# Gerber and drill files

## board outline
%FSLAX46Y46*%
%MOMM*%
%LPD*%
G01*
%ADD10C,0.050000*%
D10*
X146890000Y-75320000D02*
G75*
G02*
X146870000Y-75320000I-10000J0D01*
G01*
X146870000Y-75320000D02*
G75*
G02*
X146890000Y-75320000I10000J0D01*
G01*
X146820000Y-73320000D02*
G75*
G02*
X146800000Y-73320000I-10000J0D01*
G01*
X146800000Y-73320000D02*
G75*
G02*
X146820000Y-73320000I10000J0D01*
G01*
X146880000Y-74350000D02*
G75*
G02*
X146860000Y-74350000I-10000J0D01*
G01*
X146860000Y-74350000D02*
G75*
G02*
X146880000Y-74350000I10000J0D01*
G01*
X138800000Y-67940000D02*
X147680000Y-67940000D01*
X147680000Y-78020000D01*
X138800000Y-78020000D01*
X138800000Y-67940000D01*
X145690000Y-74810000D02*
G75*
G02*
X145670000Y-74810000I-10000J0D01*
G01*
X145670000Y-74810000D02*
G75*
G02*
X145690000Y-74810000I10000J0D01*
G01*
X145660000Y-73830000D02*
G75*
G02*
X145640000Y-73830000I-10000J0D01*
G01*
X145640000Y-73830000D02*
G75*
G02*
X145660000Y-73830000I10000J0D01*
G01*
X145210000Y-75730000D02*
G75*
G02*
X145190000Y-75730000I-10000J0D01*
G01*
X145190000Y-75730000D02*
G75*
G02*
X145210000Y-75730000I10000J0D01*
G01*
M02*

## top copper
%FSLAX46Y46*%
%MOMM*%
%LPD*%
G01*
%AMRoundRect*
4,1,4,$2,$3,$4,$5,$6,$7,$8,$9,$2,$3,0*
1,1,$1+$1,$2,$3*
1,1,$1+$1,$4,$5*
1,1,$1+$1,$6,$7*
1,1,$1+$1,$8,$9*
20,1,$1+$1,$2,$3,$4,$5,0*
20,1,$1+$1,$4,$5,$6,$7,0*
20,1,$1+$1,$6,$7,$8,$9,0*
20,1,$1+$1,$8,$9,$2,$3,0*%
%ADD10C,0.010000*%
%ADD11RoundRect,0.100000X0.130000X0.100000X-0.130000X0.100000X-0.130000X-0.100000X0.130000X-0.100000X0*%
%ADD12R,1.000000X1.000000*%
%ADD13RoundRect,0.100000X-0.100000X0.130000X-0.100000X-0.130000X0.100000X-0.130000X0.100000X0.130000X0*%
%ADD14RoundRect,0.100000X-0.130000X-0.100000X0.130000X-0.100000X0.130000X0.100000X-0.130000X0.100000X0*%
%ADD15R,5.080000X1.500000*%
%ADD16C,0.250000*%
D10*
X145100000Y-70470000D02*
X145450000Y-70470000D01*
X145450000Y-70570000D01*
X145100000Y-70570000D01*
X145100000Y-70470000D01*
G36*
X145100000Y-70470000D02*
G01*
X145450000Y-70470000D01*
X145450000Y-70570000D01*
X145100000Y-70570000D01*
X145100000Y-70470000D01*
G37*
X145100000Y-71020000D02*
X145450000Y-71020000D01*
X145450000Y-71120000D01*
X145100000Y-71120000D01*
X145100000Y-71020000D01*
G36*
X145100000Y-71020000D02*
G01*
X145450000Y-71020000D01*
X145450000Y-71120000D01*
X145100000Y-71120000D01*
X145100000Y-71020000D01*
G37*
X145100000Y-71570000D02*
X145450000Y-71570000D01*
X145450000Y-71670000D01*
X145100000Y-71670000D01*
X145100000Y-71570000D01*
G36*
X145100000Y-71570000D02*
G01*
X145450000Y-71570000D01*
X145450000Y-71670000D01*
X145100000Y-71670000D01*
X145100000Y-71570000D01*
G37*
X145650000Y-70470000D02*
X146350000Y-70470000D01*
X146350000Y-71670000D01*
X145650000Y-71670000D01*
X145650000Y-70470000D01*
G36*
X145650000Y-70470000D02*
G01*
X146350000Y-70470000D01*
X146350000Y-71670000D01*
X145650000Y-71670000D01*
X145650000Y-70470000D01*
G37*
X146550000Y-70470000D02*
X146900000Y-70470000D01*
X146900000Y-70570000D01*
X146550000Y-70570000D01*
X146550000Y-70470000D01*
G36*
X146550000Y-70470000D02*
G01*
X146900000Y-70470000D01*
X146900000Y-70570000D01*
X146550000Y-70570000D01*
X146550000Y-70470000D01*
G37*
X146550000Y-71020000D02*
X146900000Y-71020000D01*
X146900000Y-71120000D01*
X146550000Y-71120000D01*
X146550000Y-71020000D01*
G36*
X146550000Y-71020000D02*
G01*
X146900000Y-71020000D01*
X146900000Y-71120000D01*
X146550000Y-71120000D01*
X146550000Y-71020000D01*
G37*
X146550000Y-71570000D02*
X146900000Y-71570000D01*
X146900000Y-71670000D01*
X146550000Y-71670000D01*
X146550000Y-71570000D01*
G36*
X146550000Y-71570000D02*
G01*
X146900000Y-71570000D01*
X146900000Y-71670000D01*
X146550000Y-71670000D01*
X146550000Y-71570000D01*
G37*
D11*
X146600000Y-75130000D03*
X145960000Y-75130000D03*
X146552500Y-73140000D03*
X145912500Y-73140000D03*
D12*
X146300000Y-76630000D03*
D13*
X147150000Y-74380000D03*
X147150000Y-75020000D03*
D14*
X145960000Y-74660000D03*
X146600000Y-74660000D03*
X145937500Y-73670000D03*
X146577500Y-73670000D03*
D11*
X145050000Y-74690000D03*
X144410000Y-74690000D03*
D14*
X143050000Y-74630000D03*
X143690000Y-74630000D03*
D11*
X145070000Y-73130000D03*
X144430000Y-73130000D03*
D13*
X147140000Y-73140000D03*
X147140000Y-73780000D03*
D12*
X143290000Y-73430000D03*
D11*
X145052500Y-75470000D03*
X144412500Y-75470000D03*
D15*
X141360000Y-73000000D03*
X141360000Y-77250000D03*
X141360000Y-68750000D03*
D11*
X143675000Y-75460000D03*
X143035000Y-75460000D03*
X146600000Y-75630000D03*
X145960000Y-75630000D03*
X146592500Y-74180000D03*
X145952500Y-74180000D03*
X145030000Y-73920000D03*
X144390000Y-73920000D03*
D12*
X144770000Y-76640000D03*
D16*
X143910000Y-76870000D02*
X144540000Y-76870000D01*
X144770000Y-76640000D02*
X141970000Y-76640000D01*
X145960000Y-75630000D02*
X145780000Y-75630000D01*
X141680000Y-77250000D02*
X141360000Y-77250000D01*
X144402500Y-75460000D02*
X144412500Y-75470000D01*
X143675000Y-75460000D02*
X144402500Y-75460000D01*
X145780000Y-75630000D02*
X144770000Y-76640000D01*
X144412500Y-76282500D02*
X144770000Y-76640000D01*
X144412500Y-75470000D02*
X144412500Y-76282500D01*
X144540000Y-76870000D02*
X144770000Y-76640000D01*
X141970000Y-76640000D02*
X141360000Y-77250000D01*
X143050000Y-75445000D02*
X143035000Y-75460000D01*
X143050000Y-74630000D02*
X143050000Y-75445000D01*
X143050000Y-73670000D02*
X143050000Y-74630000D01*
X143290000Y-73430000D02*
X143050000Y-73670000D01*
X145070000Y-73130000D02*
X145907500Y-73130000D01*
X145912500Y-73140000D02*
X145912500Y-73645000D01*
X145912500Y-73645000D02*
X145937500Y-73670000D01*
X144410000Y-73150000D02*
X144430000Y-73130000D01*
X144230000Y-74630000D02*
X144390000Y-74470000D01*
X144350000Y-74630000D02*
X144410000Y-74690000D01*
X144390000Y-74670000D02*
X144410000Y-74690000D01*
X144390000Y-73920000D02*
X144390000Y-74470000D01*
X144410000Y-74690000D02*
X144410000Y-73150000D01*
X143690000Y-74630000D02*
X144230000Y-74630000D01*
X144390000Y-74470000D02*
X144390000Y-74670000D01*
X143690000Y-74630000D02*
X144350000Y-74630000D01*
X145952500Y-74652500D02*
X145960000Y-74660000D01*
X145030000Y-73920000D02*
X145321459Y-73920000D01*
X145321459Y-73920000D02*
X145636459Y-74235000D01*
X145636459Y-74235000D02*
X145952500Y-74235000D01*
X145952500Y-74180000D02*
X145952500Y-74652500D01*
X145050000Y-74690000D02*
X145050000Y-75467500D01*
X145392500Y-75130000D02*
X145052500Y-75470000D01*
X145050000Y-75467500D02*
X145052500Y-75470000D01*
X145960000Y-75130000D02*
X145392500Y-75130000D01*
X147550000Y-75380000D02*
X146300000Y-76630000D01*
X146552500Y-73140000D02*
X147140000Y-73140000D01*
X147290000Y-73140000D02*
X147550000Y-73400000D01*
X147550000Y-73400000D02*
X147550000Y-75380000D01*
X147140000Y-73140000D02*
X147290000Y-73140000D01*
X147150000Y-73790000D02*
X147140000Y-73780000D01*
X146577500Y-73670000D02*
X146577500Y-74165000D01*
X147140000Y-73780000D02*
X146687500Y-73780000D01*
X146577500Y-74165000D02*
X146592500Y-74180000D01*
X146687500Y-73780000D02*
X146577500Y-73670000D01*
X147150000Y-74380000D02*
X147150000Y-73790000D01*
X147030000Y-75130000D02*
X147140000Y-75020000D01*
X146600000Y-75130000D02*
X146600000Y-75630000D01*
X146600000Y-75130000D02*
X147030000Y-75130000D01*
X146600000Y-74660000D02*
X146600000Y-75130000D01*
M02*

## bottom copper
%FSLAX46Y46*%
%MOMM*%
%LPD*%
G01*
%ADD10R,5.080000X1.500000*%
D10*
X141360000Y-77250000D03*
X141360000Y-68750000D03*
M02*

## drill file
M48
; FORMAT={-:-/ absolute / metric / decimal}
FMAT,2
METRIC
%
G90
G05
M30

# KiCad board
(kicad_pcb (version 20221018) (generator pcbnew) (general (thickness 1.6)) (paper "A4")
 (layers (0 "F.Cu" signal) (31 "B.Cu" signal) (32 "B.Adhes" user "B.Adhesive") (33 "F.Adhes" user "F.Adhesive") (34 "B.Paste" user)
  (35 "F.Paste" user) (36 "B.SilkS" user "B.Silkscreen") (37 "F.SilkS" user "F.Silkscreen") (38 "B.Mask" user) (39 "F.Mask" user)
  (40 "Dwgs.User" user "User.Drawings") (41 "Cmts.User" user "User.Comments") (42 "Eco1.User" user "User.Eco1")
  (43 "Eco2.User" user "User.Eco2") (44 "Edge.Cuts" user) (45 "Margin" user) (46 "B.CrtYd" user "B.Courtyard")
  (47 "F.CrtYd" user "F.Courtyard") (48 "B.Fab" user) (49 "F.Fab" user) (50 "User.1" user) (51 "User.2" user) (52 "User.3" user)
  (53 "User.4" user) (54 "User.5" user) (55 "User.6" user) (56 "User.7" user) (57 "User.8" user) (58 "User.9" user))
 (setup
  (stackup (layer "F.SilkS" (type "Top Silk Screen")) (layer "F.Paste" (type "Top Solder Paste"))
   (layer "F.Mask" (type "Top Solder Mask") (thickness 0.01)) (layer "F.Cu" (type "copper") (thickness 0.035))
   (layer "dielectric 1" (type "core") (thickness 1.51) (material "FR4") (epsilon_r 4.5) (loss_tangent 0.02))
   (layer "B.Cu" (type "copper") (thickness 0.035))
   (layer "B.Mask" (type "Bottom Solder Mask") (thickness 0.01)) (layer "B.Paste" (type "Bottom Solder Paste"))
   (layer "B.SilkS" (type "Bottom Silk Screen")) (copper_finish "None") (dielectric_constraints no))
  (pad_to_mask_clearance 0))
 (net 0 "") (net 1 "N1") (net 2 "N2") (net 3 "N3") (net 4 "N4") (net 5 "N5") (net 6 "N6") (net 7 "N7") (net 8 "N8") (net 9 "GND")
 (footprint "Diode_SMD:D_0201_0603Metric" (layer "F.Cu") (at 146.28 75.13 180)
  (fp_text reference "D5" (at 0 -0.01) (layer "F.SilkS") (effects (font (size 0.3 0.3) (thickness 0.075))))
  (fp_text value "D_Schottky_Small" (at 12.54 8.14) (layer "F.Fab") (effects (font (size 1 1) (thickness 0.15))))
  (pad "" smd roundrect (at -0.345 0 180) (size 0.318 0.36) (layers "F.Paste") (roundrect_rratio 0.25))
  (pad "" smd roundrect (at 0.345 0 180) (size 0.318 0.36) (layers "F.Paste") (roundrect_rratio 0.25))
  (pad "1" smd roundrect (at -0.32 0 180) (size 0.46 0.4) (layers "F.Cu" "F.Mask") (roundrect_rratio 0.25) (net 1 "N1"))
  (pad "2" smd roundrect (at 0.32 0 180) (size 0.46 0.4) (layers "F.Cu" "F.Mask") (roundrect_rratio 0.25) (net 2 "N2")))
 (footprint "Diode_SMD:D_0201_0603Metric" (layer "F.Cu") (at 146.2325 73.14 180)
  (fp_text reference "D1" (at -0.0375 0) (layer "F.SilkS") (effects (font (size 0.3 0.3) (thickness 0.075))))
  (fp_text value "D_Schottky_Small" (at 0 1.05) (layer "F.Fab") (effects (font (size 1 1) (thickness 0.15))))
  (pad "" smd roundrect (at -0.345 0 180) (size 0.318 0.36) (layers "F.Paste") (roundrect_rratio 0.25))
  (pad "" smd roundrect (at 0.345 0 180) (size 0.318 0.36) (layers "F.Paste") (roundrect_rratio 0.25))
  (pad "1" smd roundrect (at -0.32 0 180) (size 0.46 0.4) (layers "F.Cu" "F.Mask") (roundrect_rratio 0.25) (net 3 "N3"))
  (pad "2" smd roundrect (at 0.32 0 180) (size 0.46 0.4) (layers "F.Cu" "F.Mask") (roundrect_rratio 0.25) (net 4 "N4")))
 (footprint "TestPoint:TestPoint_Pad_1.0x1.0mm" (layer "F.Cu") (at 146.3 76.63)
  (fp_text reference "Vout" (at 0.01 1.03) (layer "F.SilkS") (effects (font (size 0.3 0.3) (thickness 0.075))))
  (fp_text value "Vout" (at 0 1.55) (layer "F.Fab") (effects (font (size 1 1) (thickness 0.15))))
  (pad "1" smd rect (at 0 0) (size 1 1) (layers "F.Cu" "F.Mask") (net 3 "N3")))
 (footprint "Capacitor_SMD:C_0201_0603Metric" (layer "F.Cu") (at 147.15 74.7 -90)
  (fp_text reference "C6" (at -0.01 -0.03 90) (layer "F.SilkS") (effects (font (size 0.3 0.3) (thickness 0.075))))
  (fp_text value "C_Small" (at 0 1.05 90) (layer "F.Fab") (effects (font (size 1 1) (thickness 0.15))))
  (pad "" smd roundrect (at -0.345 0 270) (size 0.318 0.36) (layers "F.Paste") (roundrect_rratio 0.25))
  (pad "" smd roundrect (at 0.345 0 270) (size 0.318 0.36) (layers "F.Paste") (roundrect_rratio 0.25))
  (pad "1" smd roundrect (at -0.32 0 270) (size 0.46 0.4) (layers "F.Cu" "F.Mask") (roundrect_rratio 0.25) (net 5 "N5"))
  (pad "2" smd roundrect (at 0.32 0 270) (size 0.46 0.4) (layers "F.Cu" "F.Mask") (roundrect_rratio 0.25) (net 1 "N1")))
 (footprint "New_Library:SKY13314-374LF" (layer "F.Cu") (at 146 71.12)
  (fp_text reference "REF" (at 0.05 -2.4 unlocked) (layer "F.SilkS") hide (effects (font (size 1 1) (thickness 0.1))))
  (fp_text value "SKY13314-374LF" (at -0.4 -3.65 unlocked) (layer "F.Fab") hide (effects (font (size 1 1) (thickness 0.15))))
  (fp_rect (start -0.9 -0.65) (end -0.55 -0.55) (stroke (width 0.01) (type solid)) (fill solid) (layer "F.Cu"))
  (fp_rect (start -0.9 -0.1) (end -0.55 0) (stroke (width 0.01) (type solid)) (fill solid) (layer "F.Cu"))
  (fp_rect (start -0.9 0.45) (end -0.55 0.55) (stroke (width 0.01) (type solid)) (fill solid) (layer "F.Cu"))
  (fp_rect (start -0.35 -0.65) (end 0.35 0.55) (stroke (width 0.01) (type solid)) (fill solid) (layer "F.Cu"))
  (fp_rect (start 0.55 -0.65) (end 0.9 -0.55) (stroke (width 0.01) (type solid)) (fill solid) (layer "F.Cu"))
  (fp_rect (start 0.55 -0.1) (end 0.9 0) (stroke (width 0.01) (type solid)) (fill solid) (layer "F.Cu"))
  (fp_rect (start 0.55 0.45) (end 0.9 0.55) (stroke (width 0.01) (type solid)) (fill solid) (layer "F.Cu")))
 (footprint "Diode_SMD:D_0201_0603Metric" (layer "F.Cu") (at 146.28 74.66)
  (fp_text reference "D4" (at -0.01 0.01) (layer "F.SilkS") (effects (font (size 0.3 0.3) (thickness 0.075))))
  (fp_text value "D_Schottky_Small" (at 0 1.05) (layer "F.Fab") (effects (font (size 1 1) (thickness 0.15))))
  (pad "" smd roundrect (at -0.345 0) (size 0.318 0.36) (layers "F.Paste") (roundrect_rratio 0.25))
  (pad "" smd roundrect (at 0.345 0) (size 0.318 0.36) (layers "F.Paste") (roundrect_rratio 0.25))
  (pad "1" smd roundrect (at -0.32 0) (size 0.46 0.4) (layers "F.Cu" "F.Mask") (roundrect_rratio 0.25) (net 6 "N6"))
  (pad "2" smd roundrect (at 0.32 0) (size 0.46 0.4) (layers "F.Cu" "F.Mask") (roundrect_rratio 0.25) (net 1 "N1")))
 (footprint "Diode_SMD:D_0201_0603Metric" (layer "F.Cu") (at 146.2575 73.67)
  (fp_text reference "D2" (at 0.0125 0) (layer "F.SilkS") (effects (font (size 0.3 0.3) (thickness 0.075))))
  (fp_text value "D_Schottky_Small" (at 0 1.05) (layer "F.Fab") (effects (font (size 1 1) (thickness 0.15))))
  (pad "" smd roundrect (at -0.345 0) (size 0.318 0.36) (layers "F.Paste") (roundrect_rratio 0.25))
  (pad "" smd roundrect (at 0.345 0) (size 0.318 0.36) (layers "F.Paste") (roundrect_rratio 0.25))
  (pad "1" smd roundrect (at -0.32 0) (size 0.46 0.4) (layers "F.Cu" "F.Mask") (roundrect_rratio 0.25) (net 4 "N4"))
  (pad "2" smd roundrect (at 0.32 0) (size 0.46 0.4) (layers "F.Cu" "F.Mask") (roundrect_rratio 0.25) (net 5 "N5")))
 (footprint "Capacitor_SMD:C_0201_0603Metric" (layer "F.Cu") (at 144.73 74.69 180)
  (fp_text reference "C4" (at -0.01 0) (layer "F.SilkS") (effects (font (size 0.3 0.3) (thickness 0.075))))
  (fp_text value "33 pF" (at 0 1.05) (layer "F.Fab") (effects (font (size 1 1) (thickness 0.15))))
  (pad "" smd roundrect (at -0.345 0 180) (size 0.318 0.36) (layers "F.Paste") (roundrect_rratio 0.25))
  (pad "" smd roundrect (at 0.345 0 180) (size 0.318 0.36) (layers "F.Paste") (roundrect_rratio 0.25))
  (pad "1" smd roundrect (at -0.32 0 180) (size 0.46 0.4) (layers "F.Cu" "F.Mask") (roundrect_rratio 0.25) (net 2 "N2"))
  (pad "2" smd roundrect (at 0.32 0 180) (size 0.46 0.4) (layers "F.Cu" "F.Mask") (roundrect_rratio 0.25) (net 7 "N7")))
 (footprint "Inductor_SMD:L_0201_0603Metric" (layer "F.Cu") (at 143.37 74.63)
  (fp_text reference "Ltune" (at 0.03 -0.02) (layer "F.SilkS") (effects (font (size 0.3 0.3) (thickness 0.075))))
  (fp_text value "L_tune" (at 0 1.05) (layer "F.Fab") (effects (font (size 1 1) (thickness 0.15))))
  (pad "" smd roundrect (at -0.345 0) (size 0.318 0.36) (layers "F.Paste") (roundrect_rratio 0.25))
  (pad "" smd roundrect (at 0.345 0) (size 0.318 0.36) (layers "F.Paste") (roundrect_rratio 0.25))
  (pad "1" smd roundrect (at -0.32 0) (size 0.46 0.4) (layers "F.Cu" "F.Mask") (roundrect_rratio 0.25) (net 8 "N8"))
  (pad "2" smd roundrect (at 0.32 0) (size 0.46 0.4) (layers "F.Cu" "F.Mask") (roundrect_rratio 0.25) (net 7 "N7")))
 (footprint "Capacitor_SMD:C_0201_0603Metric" (layer "F.Cu") (at 144.75 73.13 180)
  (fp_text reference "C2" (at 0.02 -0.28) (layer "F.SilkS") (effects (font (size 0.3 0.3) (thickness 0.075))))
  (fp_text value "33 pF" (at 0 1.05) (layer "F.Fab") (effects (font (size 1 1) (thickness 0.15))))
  (pad "" smd roundrect (at -0.345 0 180) (size 0.318 0.36) (layers "F.Paste") (roundrect_rratio 0.25))
  (pad "" smd roundrect (at 0.345 0 180) (size 0.318 0.36) (layers "F.Paste") (roundrect_rratio 0.25))
  (pad "1" smd roundrect (at -0.32 0 180) (size 0.46 0.4) (layers "F.Cu" "F.Mask") (roundrect_rratio 0.25) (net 4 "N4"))
  (pad "2" smd roundrect (at 0.32 0 180) (size 0.46 0.4) (layers "F.Cu" "F.Mask") (roundrect_rratio 0.25) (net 7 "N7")))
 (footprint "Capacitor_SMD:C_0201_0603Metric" (layer "F.Cu") (at 147.14 73.46 -90)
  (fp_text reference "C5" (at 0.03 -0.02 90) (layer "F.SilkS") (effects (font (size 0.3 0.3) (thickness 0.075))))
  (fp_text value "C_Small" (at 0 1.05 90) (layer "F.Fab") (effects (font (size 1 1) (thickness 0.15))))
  (pad "" smd roundrect (at -0.345 0 270) (size 0.318 0.36) (layers "F.Paste") (roundrect_rratio 0.25))
  (pad "" smd roundrect (at 0.345 0 270) (size 0.318 0.36) (layers "F.Paste") (roundrect_rratio 0.25))
  (pad "1" smd roundrect (at -0.32 0 270) (size 0.46 0.4) (layers "F.Cu" "F.Mask") (roundrect_rratio 0.25) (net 3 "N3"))
  (pad "2" smd roundrect (at 0.32 0 270) (size 0.46 0.4) (layers "F.Cu" "F.Mask") (roundrect_rratio 0.25) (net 5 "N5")))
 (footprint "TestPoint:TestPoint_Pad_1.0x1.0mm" (layer "F.Cu") (at 143.29 73.43)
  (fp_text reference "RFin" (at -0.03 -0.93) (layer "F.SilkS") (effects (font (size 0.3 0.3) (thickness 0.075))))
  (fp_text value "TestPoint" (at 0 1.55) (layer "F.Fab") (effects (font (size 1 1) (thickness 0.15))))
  (pad "1" smd rect (at 0 0) (size 1 1) (layers "F.Cu" "F.Mask") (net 8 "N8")))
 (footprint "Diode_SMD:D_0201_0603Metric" (layer "F.Cu") (at 144.7325 75.47 180)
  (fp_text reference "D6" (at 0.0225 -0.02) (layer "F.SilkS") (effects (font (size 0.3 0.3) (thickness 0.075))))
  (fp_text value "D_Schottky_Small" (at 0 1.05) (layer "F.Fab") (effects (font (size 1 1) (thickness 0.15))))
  (pad "" smd roundrect (at -0.345 0 180) (size 0.318 0.36) (layers "F.Paste") (roundrect_rratio 0.25))
  (pad "" smd roundrect (at 0.345 0 180) (size 0.318 0.36) (layers "F.Paste") (roundrect_rratio 0.25))
  (pad "1" smd roundrect (at -0.32 0 180) (size 0.46 0.4) (layers "F.Cu" "F.Mask") (roundrect_rratio 0.25) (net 2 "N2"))
  (pad "2" smd roundrect (at 0.32 0 180) (size 0.46 0.4) (layers "F.Cu" "F.Mask") (roundrect_rratio 0.25) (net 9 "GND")))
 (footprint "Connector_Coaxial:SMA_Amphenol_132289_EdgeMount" (layer "F.Cu") (at 141.36 73 180)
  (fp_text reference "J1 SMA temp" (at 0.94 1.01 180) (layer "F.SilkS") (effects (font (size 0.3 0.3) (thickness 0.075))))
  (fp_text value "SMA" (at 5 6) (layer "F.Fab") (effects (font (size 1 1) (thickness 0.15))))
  (pad "1" smd rect (at 0 0 270) (size 1.5 5.08) (layers "F.Cu" "F.Paste" "F.Mask") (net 8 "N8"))
  (pad "2" smd rect (at 0 -4.25 270) (size 1.5 5.08) (layers "F.Cu" "F.Paste" "F.Mask") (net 9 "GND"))
  (pad "2" smd rect (at 0 -4.25 270) (size 1.5 5.08) (layers "B.Cu" "B.Paste" "B.Mask") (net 9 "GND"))
  (pad "2" smd rect (at 0 4.25 270) (size 1.5 5.08) (layers "F.Cu" "F.Paste" "F.Mask") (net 9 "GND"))
  (pad "2" smd rect (at 0 4.25 270) (size 1.5 5.08) (layers "B.Cu" "B.Paste" "B.Mask") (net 9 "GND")))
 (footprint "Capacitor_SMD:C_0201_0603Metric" (layer "F.Cu") (at 143.355 75.46 180)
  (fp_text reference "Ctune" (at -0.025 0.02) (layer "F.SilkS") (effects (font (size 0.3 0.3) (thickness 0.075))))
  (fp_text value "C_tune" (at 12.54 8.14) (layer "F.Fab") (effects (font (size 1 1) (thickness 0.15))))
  (pad "" smd roundrect (at -0.345 0 180) (size 0.318 0.36) (layers "F.Paste") (roundrect_rratio 0.25))
  (pad "" smd roundrect (at 0.345 0 180) (size 0.318 0.36) (layers "F.Paste") (roundrect_rratio 0.25))
  (pad "1" smd roundrect (at -0.32 0 180) (size 0.46 0.4) (layers "F.Cu" "F.Mask") (roundrect_rratio 0.25) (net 9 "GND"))
  (pad "2" smd roundrect (at 0.32 0 180) (size 0.46 0.4) (layers "F.Cu" "F.Mask") (roundrect_rratio 0.25) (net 8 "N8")))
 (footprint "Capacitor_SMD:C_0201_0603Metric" (layer "F.Cu") (at 146.28 75.63 180)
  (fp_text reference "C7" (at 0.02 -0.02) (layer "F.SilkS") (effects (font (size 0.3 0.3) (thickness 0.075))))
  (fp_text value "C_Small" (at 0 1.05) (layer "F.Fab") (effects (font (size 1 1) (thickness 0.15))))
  (pad "" smd roundrect (at -0.345 0 180) (size 0.318 0.36) (layers "F.Paste") (roundrect_rratio 0.25))
  (pad "" smd roundrect (at 0.345 0 180) (size 0.318 0.36) (layers "F.Paste") (roundrect_rratio 0.25))
  (pad "1" smd roundrect (at -0.32 0 180) (size 0.46 0.4) (layers "F.Cu" "F.Mask") (roundrect_rratio 0.25) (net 1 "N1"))
  (pad "2" smd roundrect (at 0.32 0 180) (size 0.46 0.4) (layers "F.Cu" "F.Mask") (roundrect_rratio 0.25) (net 9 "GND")))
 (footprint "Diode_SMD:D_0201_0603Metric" (layer "F.Cu") (at 146.2725 74.18 180)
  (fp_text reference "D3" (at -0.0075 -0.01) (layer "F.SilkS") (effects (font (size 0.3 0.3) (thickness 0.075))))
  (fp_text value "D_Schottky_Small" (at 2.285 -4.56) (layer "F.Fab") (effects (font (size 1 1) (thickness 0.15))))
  (pad "" smd roundrect (at -0.345 0 180) (size 0.318 0.36) (layers "F.Paste") (roundrect_rratio 0.25))
  (pad "" smd roundrect (at 0.345 0 180) (size 0.318 0.36) (layers "F.Paste") (roundrect_rratio 0.25))
  (pad "1" smd roundrect (at -0.32 0 180) (size 0.46 0.4) (layers "F.Cu" "F.Mask") (roundrect_rratio 0.25) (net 5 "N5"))
  (pad "2" smd roundrect (at 0.32 0 180) (size 0.46 0.4) (layers "F.Cu" "F.Mask") (roundrect_rratio 0.25) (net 6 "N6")))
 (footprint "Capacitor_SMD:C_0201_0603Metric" (layer "F.Cu") (at 144.71 73.92 180)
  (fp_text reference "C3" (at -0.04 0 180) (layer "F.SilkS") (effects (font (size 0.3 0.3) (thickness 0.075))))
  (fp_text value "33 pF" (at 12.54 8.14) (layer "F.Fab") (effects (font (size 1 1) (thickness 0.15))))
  (pad "" smd roundrect (at -0.345 0 180) (size 0.318 0.36) (layers "F.Paste") (roundrect_rratio 0.25))
  (pad "" smd roundrect (at 0.345 0 180) (size 0.318 0.36) (layers "F.Paste") (roundrect_rratio 0.25))
  (pad "1" smd roundrect (at -0.32 0 180) (size 0.46 0.4) (layers "F.Cu" "F.Mask") (roundrect_rratio 0.25) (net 6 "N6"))
  (pad "2" smd roundrect (at 0.32 0 180) (size 0.46 0.4) (layers "F.Cu" "F.Mask") (roundrect_rratio 0.25) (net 7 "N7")))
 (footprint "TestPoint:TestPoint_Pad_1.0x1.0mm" (layer "F.Cu") (at 144.77 76.64)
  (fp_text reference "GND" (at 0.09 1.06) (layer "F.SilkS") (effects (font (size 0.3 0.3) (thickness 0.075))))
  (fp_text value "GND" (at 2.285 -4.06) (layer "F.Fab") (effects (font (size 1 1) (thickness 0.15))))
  (pad "1" smd rect (at 0 0) (size 1 1) (layers "F.Cu" "F.Mask") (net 9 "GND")))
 (gr_circle (center 146.88 75.32) (end 146.88 75.33) (stroke (width 0.05) (type solid)) (fill none) (layer "Edge.Cuts"))
 (gr_circle (center 146.81 73.32) (end 146.81 73.33) (stroke (width 0.05) (type solid)) (fill none) (layer "Edge.Cuts"))
 (gr_circle (center 146.87 74.35) (end 146.87 74.36) (stroke (width 0.05) (type solid)) (fill none) (layer "Edge.Cuts"))
 (gr_rect (start 138.8 67.94) (end 147.68 78.02) (stroke (width 0.05) (type solid)) (fill none) (layer "Edge.Cuts"))
 (gr_circle (center 145.68 74.81) (end 145.68 74.82) (stroke (width 0.05) (type solid)) (fill none) (layer "Edge.Cuts"))
 (gr_circle (center 145.65 73.83) (end 145.65 73.84) (stroke (width 0.05) (type solid)) (fill none) (layer "Edge.Cuts"))
 (gr_circle (center 145.2 75.73) (end 145.2 75.74) (stroke (width 0.05) (type solid)) (fill none) (layer "Edge.Cuts"))
 (segment (start 143.91 76.87) (end 144.54 76.87) (width 0.25) (layer "F.Cu") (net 9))
 (segment (start 144.77 76.64) (end 141.97 76.64) (width 0.25) (layer "F.Cu") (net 9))
 (segment (start 145.96 75.63) (end 145.78 75.63) (width 0.25) (layer "F.Cu") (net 9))
 (segment (start 141.68 77.25) (end 141.36 77.25) (width 0.25) (layer "F.Cu") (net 9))
 (segment (start 144.4025 75.46) (end 144.4125 75.47) (width 0.25) (layer "F.Cu") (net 9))
 (segment (start 143.675 75.46) (end 144.4025 75.46) (width 0.25) (layer "F.Cu") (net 9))
 (segment (start 145.78 75.63) (end 144.77 76.64) (width 0.25) (layer "F.Cu") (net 9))
 (segment (start 144.4125 76.2825) (end 144.77 76.64) (width 0.25) (layer "F.Cu") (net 9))
 (segment (start 144.4125 75.47) (end 144.4125 76.2825) (width 0.25) (layer "F.Cu") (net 9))
 (segment (start 144.54 76.87) (end 144.77 76.64) (width 0.25) (layer "F.Cu") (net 9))
 (segment (start 141.97 76.64) (end 141.36 77.25) (width 0.25) (layer "F.Cu") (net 9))
 (segment (start 143.05 75.445) (end 143.035 75.46) (width 0.25) (layer "F.Cu") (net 8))
 (segment (start 143.05 74.63) (end 143.05 75.445) (width 0.25) (layer "F.Cu") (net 8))
 (segment (start 143.05 73.67) (end 143.05 74.63) (width 0.25) (layer "F.Cu") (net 8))
 (segment (start 143.29 73.43) (end 143.05 73.67) (width 0.25) (layer "F.Cu") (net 8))
 (segment (start 145.07 73.13) (end 145.9075 73.13) (width 0.25) (layer "F.Cu") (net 4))
 (segment (start 145.9125 73.14) (end 145.9125 73.645) (width 0.25) (layer "F.Cu") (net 4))
 (segment (start 145.9125 73.645) (end 145.9375 73.67) (width 0.25) (layer "F.Cu") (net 4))
 (segment (start 144.41 73.15) (end 144.43 73.13) (width 0.25) (layer "F.Cu") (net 7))
 (segment (start 144.23 74.63) (end 144.39 74.47) (width 0.25) (layer "F.Cu") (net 7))
 (segment (start 144.35 74.63) (end 144.41 74.69) (width 0.25) (layer "F.Cu") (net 7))
 (segment (start 144.39 74.67) (end 144.41 74.69) (width 0.25) (layer "F.Cu") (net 7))
 (segment (start 144.39 73.92) (end 144.39 74.47) (width 0.25) (layer "F.Cu") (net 7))
 (segment (start 144.41 74.69) (end 144.41 73.15) (width 0.25) (layer "F.Cu") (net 7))
 (segment (start 143.69 74.63) (end 144.23 74.63) (width 0.25) (layer "F.Cu") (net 7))
 (segment (start 144.39 74.47) (end 144.39 74.67) (width 0.25) (layer "F.Cu") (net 7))
 (segment (start 143.69 74.63) (end 144.35 74.63) (width 0.25) (layer "F.Cu") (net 7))
 (segment (start 145.9525 74.6525) (end 145.96 74.66) (width 0.25) (layer "F.Cu") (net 6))
 (segment (start 145.03 73.92) (end 145.321459 73.92) (width 0.25) (layer "F.Cu") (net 6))
 (segment (start 145.321459 73.92) (end 145.636459 74.235) (width 0.25) (layer "F.Cu") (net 6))
 (segment (start 145.636459 74.235) (end 145.9525 74.235) (width 0.25) (layer "F.Cu") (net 6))
 (segment (start 145.9525 74.18) (end 145.9525 74.6525) (width 0.25) (layer "F.Cu") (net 6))
 (segment (start 145.05 74.69) (end 145.05 75.4675) (width 0.25) (layer "F.Cu") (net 2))
 (segment (start 145.3925 75.13) (end 145.0525 75.47) (width 0.25) (layer "F.Cu") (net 2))
 (segment (start 145.05 75.4675) (end 145.0525 75.47) (width 0.25) (layer "F.Cu") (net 2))
 (segment (start 145.96 75.13) (end 145.3925 75.13) (width 0.25) (layer "F.Cu") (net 2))
 (segment (start 147.55 75.38) (end 146.3 76.63) (width 0.25) (layer "F.Cu") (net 3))
 (segment (start 146.5525 73.14) (end 147.14 73.14) (width 0.25) (layer "F.Cu") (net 3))
 (segment (start 147.29 73.14) (end 147.55 73.4) (width 0.25) (layer "F.Cu") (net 3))
 (segment (start 147.55 73.4) (end 147.55 75.38) (width 0.25) (layer "F.Cu") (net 3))
 (segment (start 147.14 73.14) (end 147.29 73.14) (width 0.25) (layer "F.Cu") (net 3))
 (segment (start 147.15 73.79) (end 147.14 73.78) (width 0.25) (layer "F.Cu") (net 5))
 (segment (start 146.5775 73.67) (end 146.5775 74.165) (width 0.25) (layer "F.Cu") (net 5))
 (segment (start 147.14 73.78) (end 146.6875 73.78) (width 0.25) (layer "F.Cu") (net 5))
 (segment (start 146.5775 74.165) (end 146.5925 74.18) (width 0.25) (layer "F.Cu") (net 5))
 (segment (start 146.6875 73.78) (end 146.5775 73.67) (width 0.25) (layer "F.Cu") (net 5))
 (segment (start 147.15 74.38) (end 147.15 73.79) (width 0.25) (layer "F.Cu") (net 5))
 (segment (start 147.03 75.13) (end 147.14 75.02) (width 0.25) (layer "F.Cu") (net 1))
 (segment (start 146.6 75.13) (end 146.6 75.63) (width 0.25) (layer "F.Cu") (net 1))
 (segment (start 146.6 75.13) (end 147.03 75.13) (width 0.25) (layer "F.Cu") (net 1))
 (segment (start 146.6 74.66) (end 146.6 75.13) (width 0.25) (layer "F.Cu") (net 1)))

